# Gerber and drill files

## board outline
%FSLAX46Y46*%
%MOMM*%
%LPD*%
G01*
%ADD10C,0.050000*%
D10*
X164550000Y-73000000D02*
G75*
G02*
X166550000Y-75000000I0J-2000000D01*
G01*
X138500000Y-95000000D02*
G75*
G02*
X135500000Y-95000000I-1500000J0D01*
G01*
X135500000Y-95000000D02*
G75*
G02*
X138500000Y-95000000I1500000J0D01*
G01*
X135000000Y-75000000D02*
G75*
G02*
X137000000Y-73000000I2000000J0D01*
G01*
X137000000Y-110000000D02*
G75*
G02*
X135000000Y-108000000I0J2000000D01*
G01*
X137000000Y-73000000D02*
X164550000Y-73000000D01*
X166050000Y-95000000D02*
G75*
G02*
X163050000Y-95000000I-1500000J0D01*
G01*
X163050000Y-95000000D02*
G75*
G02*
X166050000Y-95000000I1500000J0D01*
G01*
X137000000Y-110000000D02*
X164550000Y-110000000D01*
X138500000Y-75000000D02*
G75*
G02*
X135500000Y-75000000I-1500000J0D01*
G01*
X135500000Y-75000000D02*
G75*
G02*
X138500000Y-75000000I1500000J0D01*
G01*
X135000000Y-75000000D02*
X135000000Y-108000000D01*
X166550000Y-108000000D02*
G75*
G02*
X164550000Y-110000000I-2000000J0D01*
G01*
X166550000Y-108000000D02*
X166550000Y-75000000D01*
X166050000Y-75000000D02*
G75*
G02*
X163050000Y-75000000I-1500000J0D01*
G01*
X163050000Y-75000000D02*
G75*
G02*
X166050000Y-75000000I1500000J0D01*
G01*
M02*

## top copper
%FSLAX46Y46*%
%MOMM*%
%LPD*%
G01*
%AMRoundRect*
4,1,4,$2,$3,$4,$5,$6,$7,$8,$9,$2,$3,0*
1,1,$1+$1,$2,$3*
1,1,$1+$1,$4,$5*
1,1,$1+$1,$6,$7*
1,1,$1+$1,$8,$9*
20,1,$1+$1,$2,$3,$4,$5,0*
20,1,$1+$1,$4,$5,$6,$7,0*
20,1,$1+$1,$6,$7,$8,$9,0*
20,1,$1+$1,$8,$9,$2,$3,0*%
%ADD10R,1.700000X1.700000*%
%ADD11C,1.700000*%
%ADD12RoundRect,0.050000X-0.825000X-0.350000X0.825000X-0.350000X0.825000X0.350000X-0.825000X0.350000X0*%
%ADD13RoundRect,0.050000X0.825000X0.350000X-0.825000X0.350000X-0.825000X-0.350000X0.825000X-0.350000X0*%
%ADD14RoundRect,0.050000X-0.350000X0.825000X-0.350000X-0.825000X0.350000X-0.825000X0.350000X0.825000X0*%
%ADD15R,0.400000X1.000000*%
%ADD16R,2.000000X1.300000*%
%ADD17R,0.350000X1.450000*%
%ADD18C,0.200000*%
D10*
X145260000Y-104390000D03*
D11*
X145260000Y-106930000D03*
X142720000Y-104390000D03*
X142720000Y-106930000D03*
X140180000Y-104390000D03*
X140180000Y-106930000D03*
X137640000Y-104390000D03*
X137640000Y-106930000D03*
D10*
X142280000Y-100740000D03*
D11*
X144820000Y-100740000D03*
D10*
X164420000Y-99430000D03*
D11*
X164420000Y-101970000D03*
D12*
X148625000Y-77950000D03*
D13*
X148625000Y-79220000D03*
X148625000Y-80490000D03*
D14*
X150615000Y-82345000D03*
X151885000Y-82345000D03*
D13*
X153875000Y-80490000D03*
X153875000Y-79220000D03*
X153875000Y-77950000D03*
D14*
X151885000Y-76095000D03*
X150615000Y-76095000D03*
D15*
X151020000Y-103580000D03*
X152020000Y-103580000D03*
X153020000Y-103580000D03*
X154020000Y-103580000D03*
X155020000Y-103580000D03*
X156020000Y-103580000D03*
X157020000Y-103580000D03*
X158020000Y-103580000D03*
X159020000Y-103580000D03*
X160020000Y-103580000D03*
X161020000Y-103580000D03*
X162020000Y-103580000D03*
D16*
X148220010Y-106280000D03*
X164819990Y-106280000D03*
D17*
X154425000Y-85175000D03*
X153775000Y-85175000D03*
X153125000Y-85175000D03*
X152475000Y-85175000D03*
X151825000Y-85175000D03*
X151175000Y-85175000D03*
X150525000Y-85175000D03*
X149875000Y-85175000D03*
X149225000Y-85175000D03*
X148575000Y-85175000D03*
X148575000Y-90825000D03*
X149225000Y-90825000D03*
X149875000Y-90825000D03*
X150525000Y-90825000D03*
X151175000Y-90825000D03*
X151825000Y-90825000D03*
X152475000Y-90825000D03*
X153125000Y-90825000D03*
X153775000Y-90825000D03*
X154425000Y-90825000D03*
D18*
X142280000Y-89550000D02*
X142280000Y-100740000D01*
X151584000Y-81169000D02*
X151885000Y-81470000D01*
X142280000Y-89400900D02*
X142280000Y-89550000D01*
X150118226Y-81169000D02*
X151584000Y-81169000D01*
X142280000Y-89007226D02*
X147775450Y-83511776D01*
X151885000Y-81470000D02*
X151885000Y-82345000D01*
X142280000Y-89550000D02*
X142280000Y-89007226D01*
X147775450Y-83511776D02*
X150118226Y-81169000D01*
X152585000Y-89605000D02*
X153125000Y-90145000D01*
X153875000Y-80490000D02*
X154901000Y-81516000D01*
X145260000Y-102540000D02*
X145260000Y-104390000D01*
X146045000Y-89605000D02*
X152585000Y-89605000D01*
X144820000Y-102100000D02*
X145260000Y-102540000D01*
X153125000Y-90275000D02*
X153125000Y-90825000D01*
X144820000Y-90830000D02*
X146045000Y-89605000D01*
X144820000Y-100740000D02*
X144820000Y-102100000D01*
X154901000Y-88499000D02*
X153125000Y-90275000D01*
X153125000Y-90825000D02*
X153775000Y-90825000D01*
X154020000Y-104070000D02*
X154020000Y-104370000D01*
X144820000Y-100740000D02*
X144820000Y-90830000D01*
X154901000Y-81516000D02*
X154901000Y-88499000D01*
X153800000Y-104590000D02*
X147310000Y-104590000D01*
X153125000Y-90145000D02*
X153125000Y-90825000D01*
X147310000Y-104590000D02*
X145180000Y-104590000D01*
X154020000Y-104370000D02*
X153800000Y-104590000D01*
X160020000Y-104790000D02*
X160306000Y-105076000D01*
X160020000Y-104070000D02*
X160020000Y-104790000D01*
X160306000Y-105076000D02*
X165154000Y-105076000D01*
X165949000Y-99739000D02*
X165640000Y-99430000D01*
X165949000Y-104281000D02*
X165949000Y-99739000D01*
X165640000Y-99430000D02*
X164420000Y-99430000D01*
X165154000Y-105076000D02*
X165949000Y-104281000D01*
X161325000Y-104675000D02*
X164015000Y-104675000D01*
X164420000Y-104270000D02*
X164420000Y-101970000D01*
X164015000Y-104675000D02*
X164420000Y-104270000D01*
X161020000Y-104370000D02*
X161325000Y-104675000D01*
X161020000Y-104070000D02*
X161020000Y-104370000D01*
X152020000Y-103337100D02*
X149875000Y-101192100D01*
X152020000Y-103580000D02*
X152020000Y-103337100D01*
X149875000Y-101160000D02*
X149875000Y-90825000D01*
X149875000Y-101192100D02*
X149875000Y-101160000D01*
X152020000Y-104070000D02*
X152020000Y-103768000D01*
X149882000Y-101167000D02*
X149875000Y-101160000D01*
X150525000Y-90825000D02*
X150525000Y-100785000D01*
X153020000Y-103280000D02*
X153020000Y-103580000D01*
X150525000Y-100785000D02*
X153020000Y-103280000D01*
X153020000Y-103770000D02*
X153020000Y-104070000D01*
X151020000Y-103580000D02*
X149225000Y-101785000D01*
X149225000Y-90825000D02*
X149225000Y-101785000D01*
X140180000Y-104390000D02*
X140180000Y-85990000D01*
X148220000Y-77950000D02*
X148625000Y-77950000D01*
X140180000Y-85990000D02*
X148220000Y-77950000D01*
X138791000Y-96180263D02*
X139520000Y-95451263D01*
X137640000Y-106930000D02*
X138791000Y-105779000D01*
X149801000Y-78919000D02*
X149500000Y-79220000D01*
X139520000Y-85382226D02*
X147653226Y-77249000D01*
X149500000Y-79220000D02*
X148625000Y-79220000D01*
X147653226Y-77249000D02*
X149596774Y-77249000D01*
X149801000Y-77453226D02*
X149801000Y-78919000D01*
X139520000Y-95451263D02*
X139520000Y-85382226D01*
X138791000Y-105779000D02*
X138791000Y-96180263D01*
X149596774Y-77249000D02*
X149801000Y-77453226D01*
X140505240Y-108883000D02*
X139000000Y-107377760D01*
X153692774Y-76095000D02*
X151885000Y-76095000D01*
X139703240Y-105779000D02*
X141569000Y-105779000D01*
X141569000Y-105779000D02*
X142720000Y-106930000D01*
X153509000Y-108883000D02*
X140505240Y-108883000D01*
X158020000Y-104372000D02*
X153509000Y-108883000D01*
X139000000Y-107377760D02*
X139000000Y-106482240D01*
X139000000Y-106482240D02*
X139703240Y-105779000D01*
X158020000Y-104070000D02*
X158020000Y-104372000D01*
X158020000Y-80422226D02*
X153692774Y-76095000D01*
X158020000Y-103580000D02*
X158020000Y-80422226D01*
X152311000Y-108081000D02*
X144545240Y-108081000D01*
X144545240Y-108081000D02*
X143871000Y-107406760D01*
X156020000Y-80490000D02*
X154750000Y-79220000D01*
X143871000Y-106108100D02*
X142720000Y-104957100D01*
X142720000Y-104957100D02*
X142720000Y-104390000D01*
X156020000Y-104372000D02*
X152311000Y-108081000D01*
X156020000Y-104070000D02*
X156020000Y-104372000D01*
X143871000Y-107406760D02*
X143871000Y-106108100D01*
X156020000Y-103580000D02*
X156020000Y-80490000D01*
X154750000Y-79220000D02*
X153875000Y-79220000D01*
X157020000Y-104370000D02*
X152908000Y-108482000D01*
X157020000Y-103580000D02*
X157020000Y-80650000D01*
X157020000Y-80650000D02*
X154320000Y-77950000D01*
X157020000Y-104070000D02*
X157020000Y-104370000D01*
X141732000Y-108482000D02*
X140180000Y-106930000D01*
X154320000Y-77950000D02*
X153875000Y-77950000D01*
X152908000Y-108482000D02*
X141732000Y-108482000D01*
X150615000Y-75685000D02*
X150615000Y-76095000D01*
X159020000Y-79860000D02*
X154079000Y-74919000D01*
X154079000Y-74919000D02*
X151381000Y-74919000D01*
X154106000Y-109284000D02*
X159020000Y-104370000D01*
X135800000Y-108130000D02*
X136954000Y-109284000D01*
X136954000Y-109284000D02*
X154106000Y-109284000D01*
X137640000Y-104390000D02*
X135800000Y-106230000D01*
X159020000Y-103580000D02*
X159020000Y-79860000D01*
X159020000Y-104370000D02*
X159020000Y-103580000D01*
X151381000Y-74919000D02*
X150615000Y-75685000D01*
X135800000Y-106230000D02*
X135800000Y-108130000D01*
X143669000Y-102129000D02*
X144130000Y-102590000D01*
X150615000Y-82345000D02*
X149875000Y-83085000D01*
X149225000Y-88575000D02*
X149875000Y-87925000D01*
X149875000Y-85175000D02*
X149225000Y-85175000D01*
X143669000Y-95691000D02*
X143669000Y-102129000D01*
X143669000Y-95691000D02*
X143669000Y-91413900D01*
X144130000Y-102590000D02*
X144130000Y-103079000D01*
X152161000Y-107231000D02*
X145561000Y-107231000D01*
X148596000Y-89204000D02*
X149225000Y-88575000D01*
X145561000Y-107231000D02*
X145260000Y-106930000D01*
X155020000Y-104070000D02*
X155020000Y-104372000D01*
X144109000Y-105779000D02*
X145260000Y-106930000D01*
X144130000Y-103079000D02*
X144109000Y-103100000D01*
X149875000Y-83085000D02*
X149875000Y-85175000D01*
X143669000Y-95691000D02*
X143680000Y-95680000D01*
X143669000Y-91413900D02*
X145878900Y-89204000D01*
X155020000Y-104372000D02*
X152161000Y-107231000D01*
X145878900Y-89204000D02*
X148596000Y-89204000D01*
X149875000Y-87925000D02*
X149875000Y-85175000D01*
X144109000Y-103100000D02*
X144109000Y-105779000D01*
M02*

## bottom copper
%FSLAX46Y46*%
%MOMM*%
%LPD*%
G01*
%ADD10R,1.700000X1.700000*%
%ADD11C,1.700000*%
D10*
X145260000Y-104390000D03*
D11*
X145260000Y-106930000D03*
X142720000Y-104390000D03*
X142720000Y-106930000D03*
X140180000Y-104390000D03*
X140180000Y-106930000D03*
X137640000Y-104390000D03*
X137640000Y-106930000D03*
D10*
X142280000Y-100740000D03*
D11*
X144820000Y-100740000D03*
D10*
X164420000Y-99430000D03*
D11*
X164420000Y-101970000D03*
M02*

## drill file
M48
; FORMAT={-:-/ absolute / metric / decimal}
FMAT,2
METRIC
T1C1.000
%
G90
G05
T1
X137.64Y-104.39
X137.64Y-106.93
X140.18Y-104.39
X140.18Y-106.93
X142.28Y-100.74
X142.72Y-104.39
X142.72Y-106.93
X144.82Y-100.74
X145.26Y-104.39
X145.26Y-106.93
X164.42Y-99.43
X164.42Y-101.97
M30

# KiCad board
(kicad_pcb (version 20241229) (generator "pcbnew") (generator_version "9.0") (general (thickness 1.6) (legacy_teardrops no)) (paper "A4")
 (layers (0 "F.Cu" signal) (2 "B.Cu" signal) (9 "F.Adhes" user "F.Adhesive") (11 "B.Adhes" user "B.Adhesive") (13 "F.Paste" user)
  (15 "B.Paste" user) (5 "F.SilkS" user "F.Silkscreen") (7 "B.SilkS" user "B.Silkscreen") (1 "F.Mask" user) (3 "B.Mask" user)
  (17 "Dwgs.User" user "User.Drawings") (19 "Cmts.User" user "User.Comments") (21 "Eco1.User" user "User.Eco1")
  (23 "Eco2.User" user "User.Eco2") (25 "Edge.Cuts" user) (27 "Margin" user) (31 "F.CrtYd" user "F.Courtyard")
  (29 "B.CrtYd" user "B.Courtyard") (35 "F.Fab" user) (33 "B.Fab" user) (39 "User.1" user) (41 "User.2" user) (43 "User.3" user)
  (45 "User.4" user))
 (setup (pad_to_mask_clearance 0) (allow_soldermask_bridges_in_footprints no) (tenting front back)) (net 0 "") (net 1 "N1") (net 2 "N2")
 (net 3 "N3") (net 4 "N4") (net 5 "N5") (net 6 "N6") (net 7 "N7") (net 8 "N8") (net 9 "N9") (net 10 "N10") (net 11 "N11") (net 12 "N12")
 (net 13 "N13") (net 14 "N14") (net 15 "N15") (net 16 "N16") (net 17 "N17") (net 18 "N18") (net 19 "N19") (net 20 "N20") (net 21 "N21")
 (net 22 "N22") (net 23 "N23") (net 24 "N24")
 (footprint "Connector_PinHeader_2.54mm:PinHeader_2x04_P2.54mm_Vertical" (layer "F.Cu") (at 145.26 104.39 -90)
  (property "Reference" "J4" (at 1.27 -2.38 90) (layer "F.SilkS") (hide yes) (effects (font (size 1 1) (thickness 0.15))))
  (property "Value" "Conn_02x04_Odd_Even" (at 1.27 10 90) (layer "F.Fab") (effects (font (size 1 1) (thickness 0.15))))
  (pad "1" thru_hole rect (at 0 0 270) (size 1.7 1.7) (drill 1) (layers "*.Cu" "*.Mask") (remove_unused_layers no) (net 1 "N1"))
  (pad "2" thru_hole circle (at 2.54 0 270) (size 1.7 1.7) (drill 1) (layers "*.Cu" "*.Mask") (remove_unused_layers no) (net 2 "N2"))
  (pad "3" thru_hole circle (at 0 2.54 270) (size 1.7 1.7) (drill 1) (layers "*.Cu" "*.Mask") (remove_unused_layers no) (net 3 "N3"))
  (pad "4" thru_hole circle (at 2.54 2.54 270) (size 1.7 1.7) (drill 1) (layers "*.Cu" "*.Mask") (remove_unused_layers no) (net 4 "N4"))
  (pad "5" thru_hole circle (at 0 5.08 270) (size 1.7 1.7) (drill 1) (layers "*.Cu" "*.Mask") (remove_unused_layers no) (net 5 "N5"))
  (pad "6" thru_hole circle (at 2.54 5.08 270) (size 1.7 1.7) (drill 1) (layers "*.Cu" "*.Mask") (remove_unused_layers no) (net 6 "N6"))
  (pad "7" thru_hole circle (at 0 7.62 270) (size 1.7 1.7) (drill 1) (layers "*.Cu" "*.Mask") (remove_unused_layers no) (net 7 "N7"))
  (pad "8" thru_hole circle (at 2.54 7.62 270) (size 1.7 1.7) (drill 1) (layers "*.Cu" "*.Mask") (remove_unused_layers no) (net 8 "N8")))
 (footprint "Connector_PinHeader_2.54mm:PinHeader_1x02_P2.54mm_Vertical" (layer "F.Cu") (at 142.28 100.74 90)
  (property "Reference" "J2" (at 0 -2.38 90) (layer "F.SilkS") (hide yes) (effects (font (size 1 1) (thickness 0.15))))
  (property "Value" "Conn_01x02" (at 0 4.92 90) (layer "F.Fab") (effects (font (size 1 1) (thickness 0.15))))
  (pad "1" thru_hole rect (at 0 0 90) (size 1.7 1.7) (drill 1) (layers "*.Cu" "*.Mask") (remove_unused_layers no) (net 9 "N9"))
  (pad "2" thru_hole circle (at 0 2.54 90) (size 1.7 1.7) (drill 1) (layers "*.Cu" "*.Mask") (remove_unused_layers no) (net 1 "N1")))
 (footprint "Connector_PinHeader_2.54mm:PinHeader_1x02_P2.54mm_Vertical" (layer "F.Cu") (at 164.42 99.43)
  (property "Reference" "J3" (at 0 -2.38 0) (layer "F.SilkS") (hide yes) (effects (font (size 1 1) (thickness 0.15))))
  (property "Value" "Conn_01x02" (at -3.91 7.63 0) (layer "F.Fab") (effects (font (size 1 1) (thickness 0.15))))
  (pad "1" thru_hole rect (at 0 0) (size 1.7 1.7) (drill 1) (layers "*.Cu" "*.Mask") (remove_unused_layers no) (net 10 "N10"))
  (pad "2" thru_hole circle (at 0 2.54) (size 1.7 1.7) (drill 1) (layers "*.Cu" "*.Mask") (remove_unused_layers no) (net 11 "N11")))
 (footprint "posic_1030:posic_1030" (layer "F.Cu") (at 147.75 79.22)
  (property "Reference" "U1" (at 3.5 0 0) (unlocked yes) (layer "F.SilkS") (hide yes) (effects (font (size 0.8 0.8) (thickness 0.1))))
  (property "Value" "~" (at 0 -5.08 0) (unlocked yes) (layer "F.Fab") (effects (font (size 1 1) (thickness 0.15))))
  (pad "1" smd roundrect (at 0.875 -1.27) (size 1.75 0.8) (layers "F.Cu" "F.Mask" "F.Paste") (roundrect_rratio 0.0625) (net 5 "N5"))
  (pad "2" smd roundrect (at 0.875 0 180) (size 1.75 0.8) (layers "F.Cu" "F.Mask" "F.Paste") (roundrect_rratio 0.0625) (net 8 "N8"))
  (pad "3" smd roundrect (at 0.875 1.27 180) (size 1.75 0.8) (layers "F.Cu" "F.Mask" "F.Paste") (roundrect_rratio 0.0625) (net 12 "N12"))
  (pad "4" smd roundrect (at 2.865 3.125 270) (size 1.75 0.8) (layers "F.Cu" "F.Mask" "F.Paste") (roundrect_rratio 0.0625) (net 2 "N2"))
  (pad "5" smd roundrect (at 4.135 3.125 270) (size 1.75 0.8) (layers "F.Cu" "F.Mask" "F.Paste") (roundrect_rratio 0.0625) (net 9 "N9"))
  (pad "6" smd roundrect (at 6.125 1.27 180) (size 1.75 0.8) (layers "F.Cu" "F.Mask" "F.Paste") (roundrect_rratio 0.0625) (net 1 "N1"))
  (pad "7" smd roundrect (at 6.125 0 180) (size 1.75 0.8) (layers "F.Cu" "F.Mask" "F.Paste") (roundrect_rratio 0.0625) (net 3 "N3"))
  (pad "8" smd roundrect (at 6.125 -1.27 180) (size 1.75 0.8) (layers "F.Cu" "F.Mask" "F.Paste") (roundrect_rratio 0.0625) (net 6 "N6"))
  (pad "9" smd roundrect (at 4.135 -3.125 270) (size 1.75 0.8) (layers "F.Cu" "F.Mask" "F.Paste") (roundrect_rratio 0.0625) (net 4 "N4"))
  (pad "10" smd roundrect (at 2.865 -3.125 270) (size 1.75 0.8) (layers "F.Cu" "F.Mask" "F.Paste") (roundrect_rratio 0.0625) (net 7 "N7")))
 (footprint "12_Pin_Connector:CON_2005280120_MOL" (layer "F.Cu") (at 156.52 106.03)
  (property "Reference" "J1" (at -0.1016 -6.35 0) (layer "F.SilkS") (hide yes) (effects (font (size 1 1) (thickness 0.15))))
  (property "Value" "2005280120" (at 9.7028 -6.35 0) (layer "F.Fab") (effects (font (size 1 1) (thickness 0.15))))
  (pad "1" smd rect (at -5.5 -2.45) (size 0.4 1) (layers "F.Cu" "F.Mask" "F.Paste") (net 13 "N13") (solder_mask_margin 0.102))
  (pad "2" smd rect (at -4.5 -2.45) (size 0.4 1) (layers "F.Cu" "F.Mask" "F.Paste") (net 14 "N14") (solder_mask_margin 0.102))
  (pad "3" smd rect (at -3.5 -2.45) (size 0.4 1) (layers "F.Cu" "F.Mask" "F.Paste") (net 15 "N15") (solder_mask_margin 0.102))
  (pad "4" smd rect (at -2.5 -2.45) (size 0.4 1) (layers "F.Cu" "F.Mask" "F.Paste") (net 1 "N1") (solder_mask_margin 0.102))
  (pad "5" smd rect (at -1.5 -2.45) (size 0.4 1) (layers "F.Cu" "F.Mask" "F.Paste") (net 2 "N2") (solder_mask_margin 0.102))
  (pad "6" smd rect (at -0.5 -2.45) (size 0.4 1) (layers "F.Cu" "F.Mask" "F.Paste") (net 3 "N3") (solder_mask_margin 0.102))
  (pad "7" smd rect (at 0.5 -2.45) (size 0.4 1) (layers "F.Cu" "F.Mask" "F.Paste") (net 6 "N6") (solder_mask_margin 0.102))
  (pad "8" smd rect (at 1.5 -2.45) (size 0.4 1) (layers "F.Cu" "F.Mask" "F.Paste") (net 4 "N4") (solder_mask_margin 0.102))
  (pad "9" smd rect (at 2.5 -2.45) (size 0.4 1) (layers "F.Cu" "F.Mask" "F.Paste") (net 7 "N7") (solder_mask_margin 0.102))
  (pad "10" smd rect (at 3.5 -2.45) (size 0.4 1) (layers "F.Cu" "F.Mask" "F.Paste") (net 10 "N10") (solder_mask_margin 0.102))
  (pad "11" smd rect (at 4.5 -2.45) (size 0.4 1) (layers "F.Cu" "F.Mask" "F.Paste") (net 11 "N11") (solder_mask_margin 0.102))
  (pad "12" smd rect (at 5.5 -2.45) (size 0.4 1) (layers "F.Cu" "F.Mask" "F.Paste") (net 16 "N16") (solder_mask_margin 0.102))
  (pad "P1" smd rect (at -8.29999 0.25) (size 2 1.3) (layers "F.Cu" "F.Mask" "F.Paste") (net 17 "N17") (solder_mask_margin 0.102))
  (pad "P2" smd rect (at 8.29999 0.25) (size 2 1.3) (layers "F.Cu" "F.Mask" "F.Paste") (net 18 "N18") (solder_mask_margin 0.102)))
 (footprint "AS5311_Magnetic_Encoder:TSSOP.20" (layer "F.Cu") (at 151.5 88 180)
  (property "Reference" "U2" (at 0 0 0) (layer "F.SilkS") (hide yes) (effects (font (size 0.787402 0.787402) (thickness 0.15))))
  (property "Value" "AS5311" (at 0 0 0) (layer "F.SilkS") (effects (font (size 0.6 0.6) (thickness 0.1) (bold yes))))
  (pad "1" smd rect (at -2.925 2.825 180) (size 0.35 1.45) (layers "F.Cu" "F.Mask" "F.Paste") (solder_mask_margin 0.102))
  (pad "2" smd rect (at -2.275 2.825 180) (size 0.35 1.45) (layers "F.Cu" "F.Mask" "F.Paste") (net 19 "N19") (solder_mask_margin 0.102))
  (pad "3" smd rect (at -1.625 2.825 180) (size 0.35 1.45) (layers "F.Cu" "F.Mask" "F.Paste") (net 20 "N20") (solder_mask_margin 0.102))
  (pad "4" smd rect (at -0.975 2.825 180) (size 0.35 1.45) (layers "F.Cu" "F.Mask" "F.Paste") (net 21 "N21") (solder_mask_margin 0.102))
  (pad "5" smd rect (at -0.325 2.825 180) (size 0.35 1.45) (layers "F.Cu" "F.Mask" "F.Paste") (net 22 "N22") (solder_mask_margin 0.102))
  (pad "6" smd rect (at 0.325 2.825 180) (size 0.35 1.45) (layers "F.Cu" "F.Mask" "F.Paste") (solder_mask_margin 0.102))
  (pad "7" smd rect (at 0.975 2.825 180) (size 0.35 1.45) (layers "F.Cu" "F.Mask" "F.Paste") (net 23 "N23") (solder_mask_margin 0.102))
  (pad "8" smd rect (at 1.625 2.825 180) (size 0.35 1.45) (layers "F.Cu" "F.Mask" "F.Paste") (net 2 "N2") (solder_mask_margin 0.102))
  (pad "9" smd rect (at 2.275 2.825 180) (size 0.35 1.45) (layers "F.Cu" "F.Mask" "F.Paste") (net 2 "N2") (solder_mask_margin 0.102))
  (pad "10" smd rect (at 2.925 2.825 180) (size 0.35 1.45) (layers "F.Cu" "F.Mask" "F.Paste") (solder_mask_margin 0.102))
  (pad "11" smd rect (at 2.925 -2.825 180) (size 0.35 1.45) (layers "F.Cu" "F.Mask" "F.Paste") (solder_mask_margin 0.102))
  (pad "12" smd rect (at 2.275 -2.825 180) (size 0.35 1.45) (layers "F.Cu" "F.Mask" "F.Paste") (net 13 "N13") (solder_mask_margin 0.102))
  (pad "13" smd rect (at 1.625 -2.825 180) (size 0.35 1.45) (layers "F.Cu" "F.Mask" "F.Paste") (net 14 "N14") (solder_mask_margin 0.102))
  (pad "14" smd rect (at 0.975 -2.825 180) (size 0.35 1.45) (layers "F.Cu" "F.Mask" "F.Paste") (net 15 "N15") (solder_mask_margin 0.102))
  (pad "15" smd rect (at 0.325 -2.825 180) (size 0.35 1.45) (layers "F.Cu" "F.Mask" "F.Paste") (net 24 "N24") (solder_mask_margin 0.102))
  (pad "16" smd rect (at -0.325 -2.825 180) (size 0.35 1.45) (layers "F.Cu" "F.Mask" "F.Paste") (solder_mask_margin 0.102))
  (pad "17" smd rect (at -0.975 -2.825 180) (size 0.35 1.45) (layers "F.Cu" "F.Mask" "F.Paste") (solder_mask_margin 0.102))
  (pad "18" smd rect (at -1.625 -2.825 180) (size 0.35 1.45) (layers "F.Cu" "F.Mask" "F.Paste") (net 1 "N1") (solder_mask_margin 0.102))
  (pad "19" smd rect (at -2.275 -2.825 180) (size 0.35 1.45) (layers "F.Cu" "F.Mask" "F.Paste") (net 1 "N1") (solder_mask_margin 0.102))
  (pad "20" smd rect (at -2.925 -2.825 180) (size 0.35 1.45) (layers "F.Cu" "F.Mask" "F.Paste") (solder_mask_margin 0.102)))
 (gr_arc (start 164.55 73) (mid 165.964214 73.585786) (end 166.55 75) (stroke (width 0.05) (type default)) (layer "Edge.Cuts"))
 (gr_circle (center 137 95) (end 138.5 95) (stroke (width 0.05) (type solid)) (fill no) (layer "Edge.Cuts"))
 (gr_arc (start 135 75) (mid 135.585786 73.585786) (end 137 73) (stroke (width 0.05) (type default)) (layer "Edge.Cuts"))
 (gr_arc (start 137 110) (mid 135.585786 109.414214) (end 135 108) (stroke (width 0.05) (type default)) (layer "Edge.Cuts"))
 (gr_line (start 137 73) (end 164.55 73) (stroke (width 0.05) (type solid)) (layer "Edge.Cuts"))
 (gr_circle (center 164.55 95) (end 166.05 95) (stroke (width 0.05) (type solid)) (fill no) (layer "Edge.Cuts"))
 (gr_line (start 137 110) (end 164.55 110) (stroke (width 0.05) (type solid)) (layer "Edge.Cuts"))
 (gr_circle (center 137 75) (end 138.5 75) (stroke (width 0.05) (type solid)) (fill no) (layer "Edge.Cuts"))
 (gr_line (start 135 75) (end 135 108) (stroke (width 0.05) (type default)) (layer "Edge.Cuts"))
 (gr_arc (start 166.55 108) (mid 165.964214 109.414214) (end 164.55 110) (stroke (width 0.05) (type default)) (layer "Edge.Cuts"))
 (gr_line (start 166.55 108) (end 166.55 75) (stroke (width 0.05) (type default)) (layer "Edge.Cuts"))
 (gr_circle (center 164.55 75) (end 166.05 75) (stroke (width 0.05) (type solid)) (fill no) (layer "Edge.Cuts"))
 (segment (start 142.28 89.55) (end 142.28 100.74) (width 0.2) (layer "F.Cu") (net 9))
 (segment (start 151.584 81.169) (end 151.885 81.47) (width 0.2) (layer "F.Cu") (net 9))
 (segment (start 142.28 89.4009) (end 142.28 89.55) (width 0.2) (layer "F.Cu") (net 9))
 (segment (start 150.118226 81.169) (end 151.584 81.169) (width 0.2) (layer "F.Cu") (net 9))
 (segment (start 142.28 89.007226) (end 147.77545 83.511776) (width 0.2) (layer "F.Cu") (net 9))
 (segment (start 151.885 81.47) (end 151.885 82.345) (width 0.2) (layer "F.Cu") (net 9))
 (segment (start 142.28 89.55) (end 142.28 89.007226) (width 0.2) (layer "F.Cu") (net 9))
 (segment (start 147.77545 83.511776) (end 150.118226 81.169) (width 0.2) (layer "F.Cu") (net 9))
 (segment (start 152.585 89.605) (end 153.125 90.145) (width 0.2) (layer "F.Cu") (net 1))
 (segment (start 153.875 80.49) (end 154.901 81.516) (width 0.2) (layer "F.Cu") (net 1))
 (segment (start 145.26 102.54) (end 145.26 104.39) (width 0.2) (layer "F.Cu") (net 1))
 (segment (start 146.045 89.605) (end 152.585 89.605) (width 0.2) (layer "F.Cu") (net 1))
 (segment (start 144.82 102.1) (end 145.26 102.54) (width 0.2) (layer "F.Cu") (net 1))
 (segment (start 153.125 90.275) (end 153.125 90.825) (width 0.2) (layer "F.Cu") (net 1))
 (segment (start 144.82 90.83) (end 146.045 89.605) (width 0.2) (layer "F.Cu") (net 1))
 (segment (start 144.82 100.74) (end 144.82 102.1) (width 0.2) (layer "F.Cu") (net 1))
 (segment (start 154.901 88.499) (end 153.125 90.275) (width 0.2) (layer "F.Cu") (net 1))
 (segment (start 153.125 90.825) (end 153.775 90.825) (width 0.2) (layer "F.Cu") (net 1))
 (segment (start 154.02 104.07) (end 154.02 104.37) (width 0.2) (layer "F.Cu") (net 1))
 (segment (start 144.82 100.74) (end 144.82 90.83) (width 0.2) (layer "F.Cu") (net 1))
 (segment (start 154.901 81.516) (end 154.901 88.499) (width 0.2) (layer "F.Cu") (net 1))
 (segment (start 153.8 104.59) (end 147.31 104.59) (width 0.2) (layer "F.Cu") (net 1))
 (segment (start 153.125 90.145) (end 153.125 90.825) (width 0.2) (layer "F.Cu") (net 1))
 (segment (start 147.31 104.59) (end 145.18 104.59) (width 0.2) (layer "F.Cu") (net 1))
 (segment (start 154.02 104.37) (end 153.8 104.59) (width 0.2) (layer "F.Cu") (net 1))
 (segment (start 160.02 104.79) (end 160.306 105.076) (width 0.2) (layer "F.Cu") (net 10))
 (segment (start 160.02 104.07) (end 160.02 104.79) (width 0.2) (layer "F.Cu") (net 10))
 (segment (start 160.306 105.076) (end 165.154 105.076) (width 0.2) (layer "F.Cu") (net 10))
 (segment (start 165.949 99.739) (end 165.64 99.43) (width 0.2) (layer "F.Cu") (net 10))
 (segment (start 165.949 104.281) (end 165.949 99.739) (width 0.2) (layer "F.Cu") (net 10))
 (segment (start 165.64 99.43) (end 164.42 99.43) (width 0.2) (layer "F.Cu") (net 10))
 (segment (start 165.154 105.076) (end 165.949 104.281) (width 0.2) (layer "F.Cu") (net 10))
 (segment (start 161.325 104.675) (end 164.015 104.675) (width 0.2) (layer "F.Cu") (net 11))
 (segment (start 164.42 104.27) (end 164.42 101.97) (width 0.2) (layer "F.Cu") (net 11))
 (segment (start 164.015 104.675) (end 164.42 104.27) (width 0.2) (layer "F.Cu") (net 11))
 (segment (start 161.02 104.37) (end 161.325 104.675) (width 0.2) (layer "F.Cu") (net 11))
 (segment (start 161.02 104.07) (end 161.02 104.37) (width 0.2) (layer "F.Cu") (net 11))
 (segment (start 152.02 103.3371) (end 149.875 101.1921) (width 0.2) (layer "F.Cu") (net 14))
 (segment (start 152.02 103.58) (end 152.02 103.3371) (width 0.2) (layer "F.Cu") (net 14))
 (segment (start 149.875 101.16) (end 149.875 90.825) (width 0.2) (layer "F.Cu") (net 14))
 (segment (start 149.875 101.1921) (end 149.875 101.16) (width 0.2) (layer "F.Cu") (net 14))
 (segment (start 152.02 104.07) (end 152.02 103.768) (width 0.2) (layer "F.Cu") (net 14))
 (segment (start 149.882 101.167) (end 149.875 101.16) (width 0.2) (layer "F.Cu") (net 14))
 (segment (start 150.525 90.825) (end 150.525 100.785) (width 0.2) (layer "F.Cu") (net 15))
 (segment (start 153.02 103.28) (end 153.02 103.58) (width 0.2) (layer "F.Cu") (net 15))
 (segment (start 150.525 100.785) (end 153.02 103.28) (width 0.2) (layer "F.Cu") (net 15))
 (segment (start 153.02 103.77) (end 153.02 104.07) (width 0.2) (layer "F.Cu") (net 15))
 (segment (start 151.02 103.58) (end 149.225 101.785) (width 0.2) (layer "F.Cu") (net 13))
 (segment (start 149.225 90.825) (end 149.225 101.785) (width 0.2) (layer "F.Cu") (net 13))
 (segment (start 140.18 104.39) (end 140.18 85.99) (width 0.2) (layer "F.Cu") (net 5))
 (segment (start 148.22 77.95) (end 148.625 77.95) (width 0.2) (layer "F.Cu") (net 5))
 (segment (start 140.18 85.99) (end 148.22 77.95) (width 0.2) (layer "F.Cu") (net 5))
 (segment (start 138.791 96.180263) (end 139.52 95.451263) (width 0.2) (layer "F.Cu") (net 8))
 (segment (start 137.64 106.93) (end 138.791 105.779) (width 0.2) (layer "F.Cu") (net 8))
 (segment (start 149.801 78.919) (end 149.5 79.22) (width 0.2) (layer "F.Cu") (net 8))
 (segment (start 139.52 85.382226) (end 147.653226 77.249) (width 0.2) (layer "F.Cu") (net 8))
 (segment (start 149.5 79.22) (end 148.625 79.22) (width 0.2) (layer "F.Cu") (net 8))
 (segment (start 147.653226 77.249) (end 149.596774 77.249) (width 0.2) (layer "F.Cu") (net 8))
 (segment (start 149.801 77.453226) (end 149.801 78.919) (width 0.2) (layer "F.Cu") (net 8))
 (segment (start 139.52 95.451263) (end 139.52 85.382226) (width 0.2) (layer "F.Cu") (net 8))
 (segment (start 138.791 105.779) (end 138.791 96.180263) (width 0.2) (layer "F.Cu") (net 8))
 (segment (start 149.596774 77.249) (end 149.801 77.453226) (width 0.2) (layer "F.Cu") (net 8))
 (segment (start 140.50524 108.883) (end 139 107.37776) (width 0.2) (layer "F.Cu") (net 4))
 (segment (start 153.692774 76.095) (end 151.885 76.095) (width 0.2) (layer "F.Cu") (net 4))
 (segment (start 139.70324 105.779) (end 141.569 105.779) (width 0.2) (layer "F.Cu") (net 4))
 (segment (start 141.569 105.779) (end 142.72 106.93) (width 0.2) (layer "F.Cu") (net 4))
 (segment (start 153.509 108.883) (end 140.50524 108.883) (width 0.2) (layer "F.Cu") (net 4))
 (segment (start 158.02 104.372) (end 153.509 108.883) (width 0.2) (layer "F.Cu") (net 4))
 (segment (start 139 107.37776) (end 139 106.48224) (width 0.2) (layer "F.Cu") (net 4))
 (segment (start 139 106.48224) (end 139.70324 105.779) (width 0.2) (layer "F.Cu") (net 4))
 (segment (start 158.02 104.07) (end 158.02 104.372) (width 0.2) (layer "F.Cu") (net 4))
 (segment (start 158.02 80.422226) (end 153.692774 76.095) (width 0.2) (layer "F.Cu") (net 4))
 (segment (start 158.02 103.58) (end 158.02 80.422226) (width 0.2) (layer "F.Cu") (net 4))
 (segment (start 152.311 108.081) (end 144.54524 108.081) (width 0.2) (layer "F.Cu") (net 3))
 (segment (start 144.54524 108.081) (end 143.871 107.40676) (width 0.2) (layer "F.Cu") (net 3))
 (segment (start 156.02 80.49) (end 154.75 79.22) (width 0.2) (layer "F.Cu") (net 3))
 (segment (start 143.871 106.1081) (end 142.72 104.9571) (width 0.2) (layer "F.Cu") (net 3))
 (segment (start 142.72 104.9571) (end 142.72 104.39) (width 0.2) (layer "F.Cu") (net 3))
 (segment (start 156.02 104.372) (end 152.311 108.081) (width 0.2) (layer "F.Cu") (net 3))
 (segment (start 156.02 104.07) (end 156.02 104.372) (width 0.2) (layer "F.Cu") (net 3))
 (segment (start 143.871 107.40676) (end 143.871 106.1081) (width 0.2) (layer "F.Cu") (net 3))
 (segment (start 156.02 103.58) (end 156.02 80.49) (width 0.2) (layer "F.Cu") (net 3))
 (segment (start 154.75 79.22) (end 153.875 79.22) (width 0.2) (layer "F.Cu") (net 3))
 (segment (start 157.02 104.37) (end 152.908 108.482) (width 0.2) (layer "F.Cu") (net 6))
 (segment (start 157.02 103.58) (end 157.02 80.65) (width 0.2) (layer "F.Cu") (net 6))
 (segment (start 157.02 80.65) (end 154.32 77.95) (width 0.2) (layer "F.Cu") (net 6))
 (segment (start 157.02 104.07) (end 157.02 104.37) (width 0.2) (layer "F.Cu") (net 6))
 (segment (start 141.732 108.482) (end 140.18 106.93) (width 0.2) (layer "F.Cu") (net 6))
 (segment (start 154.32 77.95) (end 153.875 77.95) (width 0.2) (layer "F.Cu") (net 6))
 (segment (start 152.908 108.482) (end 141.732 108.482) (width 0.2) (layer "F.Cu") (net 6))
 (segment (start 150.615 75.685) (end 150.615 76.095) (width 0.2) (layer "F.Cu") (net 7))
 (segment (start 159.02 79.86) (end 154.079 74.919) (width 0.2) (layer "F.Cu") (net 7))
 (segment (start 154.079 74.919) (end 151.381 74.919) (width 0.2) (layer "F.Cu") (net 7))
 (segment (start 154.106 109.284) (end 159.02 104.37) (width 0.2) (layer "F.Cu") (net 7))
 (segment (start 135.8 108.13) (end 136.954 109.284) (width 0.2) (layer "F.Cu") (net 7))
 (segment (start 136.954 109.284) (end 154.106 109.284) (width 0.2) (layer "F.Cu") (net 7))
 (segment (start 137.64 104.39) (end 135.8 106.23) (width 0.2) (layer "F.Cu") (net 7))
 (segment (start 159.02 103.58) (end 159.02 79.86) (width 0.2) (layer "F.Cu") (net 7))
 (segment (start 159.02 104.37) (end 159.02 103.58) (width 0.2) (layer "F.Cu") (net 7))
 (segment (start 151.381 74.919) (end 150.615 75.685) (width 0.2) (layer "F.Cu") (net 7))
 (segment (start 135.8 106.23) (end 135.8 108.13) (width 0.2) (layer "F.Cu") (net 7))
 (segment (start 143.669 102.129) (end 144.13 102.59) (width 0.2) (layer "F.Cu") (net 2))
 (segment (start 150.615 82.345) (end 149.875 83.085) (width 0.2) (layer "F.Cu") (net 2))
 (segment (start 149.225 88.575) (end 149.875 87.925) (width 0.2) (layer "F.Cu") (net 2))
 (segment (start 149.875 85.175) (end 149.225 85.175) (width 0.2) (layer "F.Cu") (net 2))
 (segment (start 143.669 95.691) (end 143.669 102.129) (width 0.2) (layer "F.Cu") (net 2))
 (segment (start 143.669 95.691) (end 143.669 91.4139) (width 0.2) (layer "F.Cu") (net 2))
 (segment (start 144.13 102.59) (end 144.13 103.079) (width 0.2) (layer "F.Cu") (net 2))
 (segment (start 152.161 107.231) (end 145.561 107.231) (width 0.2) (layer "F.Cu") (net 2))
 (segment (start 148.596 89.204) (end 149.225 88.575) (width 0.2) (layer "F.Cu") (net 2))
 (segment (start 145.561 107.231) (end 145.26 106.93) (width 0.2) (layer "F.Cu") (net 2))
 (segment (start 155.02 104.07) (end 155.02 104.372) (width 0.2) (layer "F.Cu") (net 2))
 (segment (start 144.109 105.779) (end 145.26 106.93) (width 0.2) (layer "F.Cu") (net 2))
 (segment (start 144.13 103.079) (end 144.109 103.1) (width 0.2) (layer "F.Cu") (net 2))
 (segment (start 149.875 83.085) (end 149.875 85.175) (width 0.2) (layer "F.Cu") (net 2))
 (segment (start 143.669 95.691) (end 143.68 95.68) (width 0.2) (layer "F.Cu") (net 2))
 (segment (start 143.669 91.4139) (end 145.8789 89.204) (width 0.2) (layer "F.Cu") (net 2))
 (segment (start 155.02 104.372) (end 152.161 107.231) (width 0.2) (layer "F.Cu") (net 2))
 (segment (start 145.8789 89.204) (end 148.596 89.204) (width 0.2) (layer "F.Cu") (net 2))
 (segment (start 149.875 87.925) (end 149.875 85.175) (width 0.2) (layer "F.Cu") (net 2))
 (segment (start 144.109 103.1) (end 144.109 105.779) (width 0.2) (layer "F.Cu") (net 2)))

